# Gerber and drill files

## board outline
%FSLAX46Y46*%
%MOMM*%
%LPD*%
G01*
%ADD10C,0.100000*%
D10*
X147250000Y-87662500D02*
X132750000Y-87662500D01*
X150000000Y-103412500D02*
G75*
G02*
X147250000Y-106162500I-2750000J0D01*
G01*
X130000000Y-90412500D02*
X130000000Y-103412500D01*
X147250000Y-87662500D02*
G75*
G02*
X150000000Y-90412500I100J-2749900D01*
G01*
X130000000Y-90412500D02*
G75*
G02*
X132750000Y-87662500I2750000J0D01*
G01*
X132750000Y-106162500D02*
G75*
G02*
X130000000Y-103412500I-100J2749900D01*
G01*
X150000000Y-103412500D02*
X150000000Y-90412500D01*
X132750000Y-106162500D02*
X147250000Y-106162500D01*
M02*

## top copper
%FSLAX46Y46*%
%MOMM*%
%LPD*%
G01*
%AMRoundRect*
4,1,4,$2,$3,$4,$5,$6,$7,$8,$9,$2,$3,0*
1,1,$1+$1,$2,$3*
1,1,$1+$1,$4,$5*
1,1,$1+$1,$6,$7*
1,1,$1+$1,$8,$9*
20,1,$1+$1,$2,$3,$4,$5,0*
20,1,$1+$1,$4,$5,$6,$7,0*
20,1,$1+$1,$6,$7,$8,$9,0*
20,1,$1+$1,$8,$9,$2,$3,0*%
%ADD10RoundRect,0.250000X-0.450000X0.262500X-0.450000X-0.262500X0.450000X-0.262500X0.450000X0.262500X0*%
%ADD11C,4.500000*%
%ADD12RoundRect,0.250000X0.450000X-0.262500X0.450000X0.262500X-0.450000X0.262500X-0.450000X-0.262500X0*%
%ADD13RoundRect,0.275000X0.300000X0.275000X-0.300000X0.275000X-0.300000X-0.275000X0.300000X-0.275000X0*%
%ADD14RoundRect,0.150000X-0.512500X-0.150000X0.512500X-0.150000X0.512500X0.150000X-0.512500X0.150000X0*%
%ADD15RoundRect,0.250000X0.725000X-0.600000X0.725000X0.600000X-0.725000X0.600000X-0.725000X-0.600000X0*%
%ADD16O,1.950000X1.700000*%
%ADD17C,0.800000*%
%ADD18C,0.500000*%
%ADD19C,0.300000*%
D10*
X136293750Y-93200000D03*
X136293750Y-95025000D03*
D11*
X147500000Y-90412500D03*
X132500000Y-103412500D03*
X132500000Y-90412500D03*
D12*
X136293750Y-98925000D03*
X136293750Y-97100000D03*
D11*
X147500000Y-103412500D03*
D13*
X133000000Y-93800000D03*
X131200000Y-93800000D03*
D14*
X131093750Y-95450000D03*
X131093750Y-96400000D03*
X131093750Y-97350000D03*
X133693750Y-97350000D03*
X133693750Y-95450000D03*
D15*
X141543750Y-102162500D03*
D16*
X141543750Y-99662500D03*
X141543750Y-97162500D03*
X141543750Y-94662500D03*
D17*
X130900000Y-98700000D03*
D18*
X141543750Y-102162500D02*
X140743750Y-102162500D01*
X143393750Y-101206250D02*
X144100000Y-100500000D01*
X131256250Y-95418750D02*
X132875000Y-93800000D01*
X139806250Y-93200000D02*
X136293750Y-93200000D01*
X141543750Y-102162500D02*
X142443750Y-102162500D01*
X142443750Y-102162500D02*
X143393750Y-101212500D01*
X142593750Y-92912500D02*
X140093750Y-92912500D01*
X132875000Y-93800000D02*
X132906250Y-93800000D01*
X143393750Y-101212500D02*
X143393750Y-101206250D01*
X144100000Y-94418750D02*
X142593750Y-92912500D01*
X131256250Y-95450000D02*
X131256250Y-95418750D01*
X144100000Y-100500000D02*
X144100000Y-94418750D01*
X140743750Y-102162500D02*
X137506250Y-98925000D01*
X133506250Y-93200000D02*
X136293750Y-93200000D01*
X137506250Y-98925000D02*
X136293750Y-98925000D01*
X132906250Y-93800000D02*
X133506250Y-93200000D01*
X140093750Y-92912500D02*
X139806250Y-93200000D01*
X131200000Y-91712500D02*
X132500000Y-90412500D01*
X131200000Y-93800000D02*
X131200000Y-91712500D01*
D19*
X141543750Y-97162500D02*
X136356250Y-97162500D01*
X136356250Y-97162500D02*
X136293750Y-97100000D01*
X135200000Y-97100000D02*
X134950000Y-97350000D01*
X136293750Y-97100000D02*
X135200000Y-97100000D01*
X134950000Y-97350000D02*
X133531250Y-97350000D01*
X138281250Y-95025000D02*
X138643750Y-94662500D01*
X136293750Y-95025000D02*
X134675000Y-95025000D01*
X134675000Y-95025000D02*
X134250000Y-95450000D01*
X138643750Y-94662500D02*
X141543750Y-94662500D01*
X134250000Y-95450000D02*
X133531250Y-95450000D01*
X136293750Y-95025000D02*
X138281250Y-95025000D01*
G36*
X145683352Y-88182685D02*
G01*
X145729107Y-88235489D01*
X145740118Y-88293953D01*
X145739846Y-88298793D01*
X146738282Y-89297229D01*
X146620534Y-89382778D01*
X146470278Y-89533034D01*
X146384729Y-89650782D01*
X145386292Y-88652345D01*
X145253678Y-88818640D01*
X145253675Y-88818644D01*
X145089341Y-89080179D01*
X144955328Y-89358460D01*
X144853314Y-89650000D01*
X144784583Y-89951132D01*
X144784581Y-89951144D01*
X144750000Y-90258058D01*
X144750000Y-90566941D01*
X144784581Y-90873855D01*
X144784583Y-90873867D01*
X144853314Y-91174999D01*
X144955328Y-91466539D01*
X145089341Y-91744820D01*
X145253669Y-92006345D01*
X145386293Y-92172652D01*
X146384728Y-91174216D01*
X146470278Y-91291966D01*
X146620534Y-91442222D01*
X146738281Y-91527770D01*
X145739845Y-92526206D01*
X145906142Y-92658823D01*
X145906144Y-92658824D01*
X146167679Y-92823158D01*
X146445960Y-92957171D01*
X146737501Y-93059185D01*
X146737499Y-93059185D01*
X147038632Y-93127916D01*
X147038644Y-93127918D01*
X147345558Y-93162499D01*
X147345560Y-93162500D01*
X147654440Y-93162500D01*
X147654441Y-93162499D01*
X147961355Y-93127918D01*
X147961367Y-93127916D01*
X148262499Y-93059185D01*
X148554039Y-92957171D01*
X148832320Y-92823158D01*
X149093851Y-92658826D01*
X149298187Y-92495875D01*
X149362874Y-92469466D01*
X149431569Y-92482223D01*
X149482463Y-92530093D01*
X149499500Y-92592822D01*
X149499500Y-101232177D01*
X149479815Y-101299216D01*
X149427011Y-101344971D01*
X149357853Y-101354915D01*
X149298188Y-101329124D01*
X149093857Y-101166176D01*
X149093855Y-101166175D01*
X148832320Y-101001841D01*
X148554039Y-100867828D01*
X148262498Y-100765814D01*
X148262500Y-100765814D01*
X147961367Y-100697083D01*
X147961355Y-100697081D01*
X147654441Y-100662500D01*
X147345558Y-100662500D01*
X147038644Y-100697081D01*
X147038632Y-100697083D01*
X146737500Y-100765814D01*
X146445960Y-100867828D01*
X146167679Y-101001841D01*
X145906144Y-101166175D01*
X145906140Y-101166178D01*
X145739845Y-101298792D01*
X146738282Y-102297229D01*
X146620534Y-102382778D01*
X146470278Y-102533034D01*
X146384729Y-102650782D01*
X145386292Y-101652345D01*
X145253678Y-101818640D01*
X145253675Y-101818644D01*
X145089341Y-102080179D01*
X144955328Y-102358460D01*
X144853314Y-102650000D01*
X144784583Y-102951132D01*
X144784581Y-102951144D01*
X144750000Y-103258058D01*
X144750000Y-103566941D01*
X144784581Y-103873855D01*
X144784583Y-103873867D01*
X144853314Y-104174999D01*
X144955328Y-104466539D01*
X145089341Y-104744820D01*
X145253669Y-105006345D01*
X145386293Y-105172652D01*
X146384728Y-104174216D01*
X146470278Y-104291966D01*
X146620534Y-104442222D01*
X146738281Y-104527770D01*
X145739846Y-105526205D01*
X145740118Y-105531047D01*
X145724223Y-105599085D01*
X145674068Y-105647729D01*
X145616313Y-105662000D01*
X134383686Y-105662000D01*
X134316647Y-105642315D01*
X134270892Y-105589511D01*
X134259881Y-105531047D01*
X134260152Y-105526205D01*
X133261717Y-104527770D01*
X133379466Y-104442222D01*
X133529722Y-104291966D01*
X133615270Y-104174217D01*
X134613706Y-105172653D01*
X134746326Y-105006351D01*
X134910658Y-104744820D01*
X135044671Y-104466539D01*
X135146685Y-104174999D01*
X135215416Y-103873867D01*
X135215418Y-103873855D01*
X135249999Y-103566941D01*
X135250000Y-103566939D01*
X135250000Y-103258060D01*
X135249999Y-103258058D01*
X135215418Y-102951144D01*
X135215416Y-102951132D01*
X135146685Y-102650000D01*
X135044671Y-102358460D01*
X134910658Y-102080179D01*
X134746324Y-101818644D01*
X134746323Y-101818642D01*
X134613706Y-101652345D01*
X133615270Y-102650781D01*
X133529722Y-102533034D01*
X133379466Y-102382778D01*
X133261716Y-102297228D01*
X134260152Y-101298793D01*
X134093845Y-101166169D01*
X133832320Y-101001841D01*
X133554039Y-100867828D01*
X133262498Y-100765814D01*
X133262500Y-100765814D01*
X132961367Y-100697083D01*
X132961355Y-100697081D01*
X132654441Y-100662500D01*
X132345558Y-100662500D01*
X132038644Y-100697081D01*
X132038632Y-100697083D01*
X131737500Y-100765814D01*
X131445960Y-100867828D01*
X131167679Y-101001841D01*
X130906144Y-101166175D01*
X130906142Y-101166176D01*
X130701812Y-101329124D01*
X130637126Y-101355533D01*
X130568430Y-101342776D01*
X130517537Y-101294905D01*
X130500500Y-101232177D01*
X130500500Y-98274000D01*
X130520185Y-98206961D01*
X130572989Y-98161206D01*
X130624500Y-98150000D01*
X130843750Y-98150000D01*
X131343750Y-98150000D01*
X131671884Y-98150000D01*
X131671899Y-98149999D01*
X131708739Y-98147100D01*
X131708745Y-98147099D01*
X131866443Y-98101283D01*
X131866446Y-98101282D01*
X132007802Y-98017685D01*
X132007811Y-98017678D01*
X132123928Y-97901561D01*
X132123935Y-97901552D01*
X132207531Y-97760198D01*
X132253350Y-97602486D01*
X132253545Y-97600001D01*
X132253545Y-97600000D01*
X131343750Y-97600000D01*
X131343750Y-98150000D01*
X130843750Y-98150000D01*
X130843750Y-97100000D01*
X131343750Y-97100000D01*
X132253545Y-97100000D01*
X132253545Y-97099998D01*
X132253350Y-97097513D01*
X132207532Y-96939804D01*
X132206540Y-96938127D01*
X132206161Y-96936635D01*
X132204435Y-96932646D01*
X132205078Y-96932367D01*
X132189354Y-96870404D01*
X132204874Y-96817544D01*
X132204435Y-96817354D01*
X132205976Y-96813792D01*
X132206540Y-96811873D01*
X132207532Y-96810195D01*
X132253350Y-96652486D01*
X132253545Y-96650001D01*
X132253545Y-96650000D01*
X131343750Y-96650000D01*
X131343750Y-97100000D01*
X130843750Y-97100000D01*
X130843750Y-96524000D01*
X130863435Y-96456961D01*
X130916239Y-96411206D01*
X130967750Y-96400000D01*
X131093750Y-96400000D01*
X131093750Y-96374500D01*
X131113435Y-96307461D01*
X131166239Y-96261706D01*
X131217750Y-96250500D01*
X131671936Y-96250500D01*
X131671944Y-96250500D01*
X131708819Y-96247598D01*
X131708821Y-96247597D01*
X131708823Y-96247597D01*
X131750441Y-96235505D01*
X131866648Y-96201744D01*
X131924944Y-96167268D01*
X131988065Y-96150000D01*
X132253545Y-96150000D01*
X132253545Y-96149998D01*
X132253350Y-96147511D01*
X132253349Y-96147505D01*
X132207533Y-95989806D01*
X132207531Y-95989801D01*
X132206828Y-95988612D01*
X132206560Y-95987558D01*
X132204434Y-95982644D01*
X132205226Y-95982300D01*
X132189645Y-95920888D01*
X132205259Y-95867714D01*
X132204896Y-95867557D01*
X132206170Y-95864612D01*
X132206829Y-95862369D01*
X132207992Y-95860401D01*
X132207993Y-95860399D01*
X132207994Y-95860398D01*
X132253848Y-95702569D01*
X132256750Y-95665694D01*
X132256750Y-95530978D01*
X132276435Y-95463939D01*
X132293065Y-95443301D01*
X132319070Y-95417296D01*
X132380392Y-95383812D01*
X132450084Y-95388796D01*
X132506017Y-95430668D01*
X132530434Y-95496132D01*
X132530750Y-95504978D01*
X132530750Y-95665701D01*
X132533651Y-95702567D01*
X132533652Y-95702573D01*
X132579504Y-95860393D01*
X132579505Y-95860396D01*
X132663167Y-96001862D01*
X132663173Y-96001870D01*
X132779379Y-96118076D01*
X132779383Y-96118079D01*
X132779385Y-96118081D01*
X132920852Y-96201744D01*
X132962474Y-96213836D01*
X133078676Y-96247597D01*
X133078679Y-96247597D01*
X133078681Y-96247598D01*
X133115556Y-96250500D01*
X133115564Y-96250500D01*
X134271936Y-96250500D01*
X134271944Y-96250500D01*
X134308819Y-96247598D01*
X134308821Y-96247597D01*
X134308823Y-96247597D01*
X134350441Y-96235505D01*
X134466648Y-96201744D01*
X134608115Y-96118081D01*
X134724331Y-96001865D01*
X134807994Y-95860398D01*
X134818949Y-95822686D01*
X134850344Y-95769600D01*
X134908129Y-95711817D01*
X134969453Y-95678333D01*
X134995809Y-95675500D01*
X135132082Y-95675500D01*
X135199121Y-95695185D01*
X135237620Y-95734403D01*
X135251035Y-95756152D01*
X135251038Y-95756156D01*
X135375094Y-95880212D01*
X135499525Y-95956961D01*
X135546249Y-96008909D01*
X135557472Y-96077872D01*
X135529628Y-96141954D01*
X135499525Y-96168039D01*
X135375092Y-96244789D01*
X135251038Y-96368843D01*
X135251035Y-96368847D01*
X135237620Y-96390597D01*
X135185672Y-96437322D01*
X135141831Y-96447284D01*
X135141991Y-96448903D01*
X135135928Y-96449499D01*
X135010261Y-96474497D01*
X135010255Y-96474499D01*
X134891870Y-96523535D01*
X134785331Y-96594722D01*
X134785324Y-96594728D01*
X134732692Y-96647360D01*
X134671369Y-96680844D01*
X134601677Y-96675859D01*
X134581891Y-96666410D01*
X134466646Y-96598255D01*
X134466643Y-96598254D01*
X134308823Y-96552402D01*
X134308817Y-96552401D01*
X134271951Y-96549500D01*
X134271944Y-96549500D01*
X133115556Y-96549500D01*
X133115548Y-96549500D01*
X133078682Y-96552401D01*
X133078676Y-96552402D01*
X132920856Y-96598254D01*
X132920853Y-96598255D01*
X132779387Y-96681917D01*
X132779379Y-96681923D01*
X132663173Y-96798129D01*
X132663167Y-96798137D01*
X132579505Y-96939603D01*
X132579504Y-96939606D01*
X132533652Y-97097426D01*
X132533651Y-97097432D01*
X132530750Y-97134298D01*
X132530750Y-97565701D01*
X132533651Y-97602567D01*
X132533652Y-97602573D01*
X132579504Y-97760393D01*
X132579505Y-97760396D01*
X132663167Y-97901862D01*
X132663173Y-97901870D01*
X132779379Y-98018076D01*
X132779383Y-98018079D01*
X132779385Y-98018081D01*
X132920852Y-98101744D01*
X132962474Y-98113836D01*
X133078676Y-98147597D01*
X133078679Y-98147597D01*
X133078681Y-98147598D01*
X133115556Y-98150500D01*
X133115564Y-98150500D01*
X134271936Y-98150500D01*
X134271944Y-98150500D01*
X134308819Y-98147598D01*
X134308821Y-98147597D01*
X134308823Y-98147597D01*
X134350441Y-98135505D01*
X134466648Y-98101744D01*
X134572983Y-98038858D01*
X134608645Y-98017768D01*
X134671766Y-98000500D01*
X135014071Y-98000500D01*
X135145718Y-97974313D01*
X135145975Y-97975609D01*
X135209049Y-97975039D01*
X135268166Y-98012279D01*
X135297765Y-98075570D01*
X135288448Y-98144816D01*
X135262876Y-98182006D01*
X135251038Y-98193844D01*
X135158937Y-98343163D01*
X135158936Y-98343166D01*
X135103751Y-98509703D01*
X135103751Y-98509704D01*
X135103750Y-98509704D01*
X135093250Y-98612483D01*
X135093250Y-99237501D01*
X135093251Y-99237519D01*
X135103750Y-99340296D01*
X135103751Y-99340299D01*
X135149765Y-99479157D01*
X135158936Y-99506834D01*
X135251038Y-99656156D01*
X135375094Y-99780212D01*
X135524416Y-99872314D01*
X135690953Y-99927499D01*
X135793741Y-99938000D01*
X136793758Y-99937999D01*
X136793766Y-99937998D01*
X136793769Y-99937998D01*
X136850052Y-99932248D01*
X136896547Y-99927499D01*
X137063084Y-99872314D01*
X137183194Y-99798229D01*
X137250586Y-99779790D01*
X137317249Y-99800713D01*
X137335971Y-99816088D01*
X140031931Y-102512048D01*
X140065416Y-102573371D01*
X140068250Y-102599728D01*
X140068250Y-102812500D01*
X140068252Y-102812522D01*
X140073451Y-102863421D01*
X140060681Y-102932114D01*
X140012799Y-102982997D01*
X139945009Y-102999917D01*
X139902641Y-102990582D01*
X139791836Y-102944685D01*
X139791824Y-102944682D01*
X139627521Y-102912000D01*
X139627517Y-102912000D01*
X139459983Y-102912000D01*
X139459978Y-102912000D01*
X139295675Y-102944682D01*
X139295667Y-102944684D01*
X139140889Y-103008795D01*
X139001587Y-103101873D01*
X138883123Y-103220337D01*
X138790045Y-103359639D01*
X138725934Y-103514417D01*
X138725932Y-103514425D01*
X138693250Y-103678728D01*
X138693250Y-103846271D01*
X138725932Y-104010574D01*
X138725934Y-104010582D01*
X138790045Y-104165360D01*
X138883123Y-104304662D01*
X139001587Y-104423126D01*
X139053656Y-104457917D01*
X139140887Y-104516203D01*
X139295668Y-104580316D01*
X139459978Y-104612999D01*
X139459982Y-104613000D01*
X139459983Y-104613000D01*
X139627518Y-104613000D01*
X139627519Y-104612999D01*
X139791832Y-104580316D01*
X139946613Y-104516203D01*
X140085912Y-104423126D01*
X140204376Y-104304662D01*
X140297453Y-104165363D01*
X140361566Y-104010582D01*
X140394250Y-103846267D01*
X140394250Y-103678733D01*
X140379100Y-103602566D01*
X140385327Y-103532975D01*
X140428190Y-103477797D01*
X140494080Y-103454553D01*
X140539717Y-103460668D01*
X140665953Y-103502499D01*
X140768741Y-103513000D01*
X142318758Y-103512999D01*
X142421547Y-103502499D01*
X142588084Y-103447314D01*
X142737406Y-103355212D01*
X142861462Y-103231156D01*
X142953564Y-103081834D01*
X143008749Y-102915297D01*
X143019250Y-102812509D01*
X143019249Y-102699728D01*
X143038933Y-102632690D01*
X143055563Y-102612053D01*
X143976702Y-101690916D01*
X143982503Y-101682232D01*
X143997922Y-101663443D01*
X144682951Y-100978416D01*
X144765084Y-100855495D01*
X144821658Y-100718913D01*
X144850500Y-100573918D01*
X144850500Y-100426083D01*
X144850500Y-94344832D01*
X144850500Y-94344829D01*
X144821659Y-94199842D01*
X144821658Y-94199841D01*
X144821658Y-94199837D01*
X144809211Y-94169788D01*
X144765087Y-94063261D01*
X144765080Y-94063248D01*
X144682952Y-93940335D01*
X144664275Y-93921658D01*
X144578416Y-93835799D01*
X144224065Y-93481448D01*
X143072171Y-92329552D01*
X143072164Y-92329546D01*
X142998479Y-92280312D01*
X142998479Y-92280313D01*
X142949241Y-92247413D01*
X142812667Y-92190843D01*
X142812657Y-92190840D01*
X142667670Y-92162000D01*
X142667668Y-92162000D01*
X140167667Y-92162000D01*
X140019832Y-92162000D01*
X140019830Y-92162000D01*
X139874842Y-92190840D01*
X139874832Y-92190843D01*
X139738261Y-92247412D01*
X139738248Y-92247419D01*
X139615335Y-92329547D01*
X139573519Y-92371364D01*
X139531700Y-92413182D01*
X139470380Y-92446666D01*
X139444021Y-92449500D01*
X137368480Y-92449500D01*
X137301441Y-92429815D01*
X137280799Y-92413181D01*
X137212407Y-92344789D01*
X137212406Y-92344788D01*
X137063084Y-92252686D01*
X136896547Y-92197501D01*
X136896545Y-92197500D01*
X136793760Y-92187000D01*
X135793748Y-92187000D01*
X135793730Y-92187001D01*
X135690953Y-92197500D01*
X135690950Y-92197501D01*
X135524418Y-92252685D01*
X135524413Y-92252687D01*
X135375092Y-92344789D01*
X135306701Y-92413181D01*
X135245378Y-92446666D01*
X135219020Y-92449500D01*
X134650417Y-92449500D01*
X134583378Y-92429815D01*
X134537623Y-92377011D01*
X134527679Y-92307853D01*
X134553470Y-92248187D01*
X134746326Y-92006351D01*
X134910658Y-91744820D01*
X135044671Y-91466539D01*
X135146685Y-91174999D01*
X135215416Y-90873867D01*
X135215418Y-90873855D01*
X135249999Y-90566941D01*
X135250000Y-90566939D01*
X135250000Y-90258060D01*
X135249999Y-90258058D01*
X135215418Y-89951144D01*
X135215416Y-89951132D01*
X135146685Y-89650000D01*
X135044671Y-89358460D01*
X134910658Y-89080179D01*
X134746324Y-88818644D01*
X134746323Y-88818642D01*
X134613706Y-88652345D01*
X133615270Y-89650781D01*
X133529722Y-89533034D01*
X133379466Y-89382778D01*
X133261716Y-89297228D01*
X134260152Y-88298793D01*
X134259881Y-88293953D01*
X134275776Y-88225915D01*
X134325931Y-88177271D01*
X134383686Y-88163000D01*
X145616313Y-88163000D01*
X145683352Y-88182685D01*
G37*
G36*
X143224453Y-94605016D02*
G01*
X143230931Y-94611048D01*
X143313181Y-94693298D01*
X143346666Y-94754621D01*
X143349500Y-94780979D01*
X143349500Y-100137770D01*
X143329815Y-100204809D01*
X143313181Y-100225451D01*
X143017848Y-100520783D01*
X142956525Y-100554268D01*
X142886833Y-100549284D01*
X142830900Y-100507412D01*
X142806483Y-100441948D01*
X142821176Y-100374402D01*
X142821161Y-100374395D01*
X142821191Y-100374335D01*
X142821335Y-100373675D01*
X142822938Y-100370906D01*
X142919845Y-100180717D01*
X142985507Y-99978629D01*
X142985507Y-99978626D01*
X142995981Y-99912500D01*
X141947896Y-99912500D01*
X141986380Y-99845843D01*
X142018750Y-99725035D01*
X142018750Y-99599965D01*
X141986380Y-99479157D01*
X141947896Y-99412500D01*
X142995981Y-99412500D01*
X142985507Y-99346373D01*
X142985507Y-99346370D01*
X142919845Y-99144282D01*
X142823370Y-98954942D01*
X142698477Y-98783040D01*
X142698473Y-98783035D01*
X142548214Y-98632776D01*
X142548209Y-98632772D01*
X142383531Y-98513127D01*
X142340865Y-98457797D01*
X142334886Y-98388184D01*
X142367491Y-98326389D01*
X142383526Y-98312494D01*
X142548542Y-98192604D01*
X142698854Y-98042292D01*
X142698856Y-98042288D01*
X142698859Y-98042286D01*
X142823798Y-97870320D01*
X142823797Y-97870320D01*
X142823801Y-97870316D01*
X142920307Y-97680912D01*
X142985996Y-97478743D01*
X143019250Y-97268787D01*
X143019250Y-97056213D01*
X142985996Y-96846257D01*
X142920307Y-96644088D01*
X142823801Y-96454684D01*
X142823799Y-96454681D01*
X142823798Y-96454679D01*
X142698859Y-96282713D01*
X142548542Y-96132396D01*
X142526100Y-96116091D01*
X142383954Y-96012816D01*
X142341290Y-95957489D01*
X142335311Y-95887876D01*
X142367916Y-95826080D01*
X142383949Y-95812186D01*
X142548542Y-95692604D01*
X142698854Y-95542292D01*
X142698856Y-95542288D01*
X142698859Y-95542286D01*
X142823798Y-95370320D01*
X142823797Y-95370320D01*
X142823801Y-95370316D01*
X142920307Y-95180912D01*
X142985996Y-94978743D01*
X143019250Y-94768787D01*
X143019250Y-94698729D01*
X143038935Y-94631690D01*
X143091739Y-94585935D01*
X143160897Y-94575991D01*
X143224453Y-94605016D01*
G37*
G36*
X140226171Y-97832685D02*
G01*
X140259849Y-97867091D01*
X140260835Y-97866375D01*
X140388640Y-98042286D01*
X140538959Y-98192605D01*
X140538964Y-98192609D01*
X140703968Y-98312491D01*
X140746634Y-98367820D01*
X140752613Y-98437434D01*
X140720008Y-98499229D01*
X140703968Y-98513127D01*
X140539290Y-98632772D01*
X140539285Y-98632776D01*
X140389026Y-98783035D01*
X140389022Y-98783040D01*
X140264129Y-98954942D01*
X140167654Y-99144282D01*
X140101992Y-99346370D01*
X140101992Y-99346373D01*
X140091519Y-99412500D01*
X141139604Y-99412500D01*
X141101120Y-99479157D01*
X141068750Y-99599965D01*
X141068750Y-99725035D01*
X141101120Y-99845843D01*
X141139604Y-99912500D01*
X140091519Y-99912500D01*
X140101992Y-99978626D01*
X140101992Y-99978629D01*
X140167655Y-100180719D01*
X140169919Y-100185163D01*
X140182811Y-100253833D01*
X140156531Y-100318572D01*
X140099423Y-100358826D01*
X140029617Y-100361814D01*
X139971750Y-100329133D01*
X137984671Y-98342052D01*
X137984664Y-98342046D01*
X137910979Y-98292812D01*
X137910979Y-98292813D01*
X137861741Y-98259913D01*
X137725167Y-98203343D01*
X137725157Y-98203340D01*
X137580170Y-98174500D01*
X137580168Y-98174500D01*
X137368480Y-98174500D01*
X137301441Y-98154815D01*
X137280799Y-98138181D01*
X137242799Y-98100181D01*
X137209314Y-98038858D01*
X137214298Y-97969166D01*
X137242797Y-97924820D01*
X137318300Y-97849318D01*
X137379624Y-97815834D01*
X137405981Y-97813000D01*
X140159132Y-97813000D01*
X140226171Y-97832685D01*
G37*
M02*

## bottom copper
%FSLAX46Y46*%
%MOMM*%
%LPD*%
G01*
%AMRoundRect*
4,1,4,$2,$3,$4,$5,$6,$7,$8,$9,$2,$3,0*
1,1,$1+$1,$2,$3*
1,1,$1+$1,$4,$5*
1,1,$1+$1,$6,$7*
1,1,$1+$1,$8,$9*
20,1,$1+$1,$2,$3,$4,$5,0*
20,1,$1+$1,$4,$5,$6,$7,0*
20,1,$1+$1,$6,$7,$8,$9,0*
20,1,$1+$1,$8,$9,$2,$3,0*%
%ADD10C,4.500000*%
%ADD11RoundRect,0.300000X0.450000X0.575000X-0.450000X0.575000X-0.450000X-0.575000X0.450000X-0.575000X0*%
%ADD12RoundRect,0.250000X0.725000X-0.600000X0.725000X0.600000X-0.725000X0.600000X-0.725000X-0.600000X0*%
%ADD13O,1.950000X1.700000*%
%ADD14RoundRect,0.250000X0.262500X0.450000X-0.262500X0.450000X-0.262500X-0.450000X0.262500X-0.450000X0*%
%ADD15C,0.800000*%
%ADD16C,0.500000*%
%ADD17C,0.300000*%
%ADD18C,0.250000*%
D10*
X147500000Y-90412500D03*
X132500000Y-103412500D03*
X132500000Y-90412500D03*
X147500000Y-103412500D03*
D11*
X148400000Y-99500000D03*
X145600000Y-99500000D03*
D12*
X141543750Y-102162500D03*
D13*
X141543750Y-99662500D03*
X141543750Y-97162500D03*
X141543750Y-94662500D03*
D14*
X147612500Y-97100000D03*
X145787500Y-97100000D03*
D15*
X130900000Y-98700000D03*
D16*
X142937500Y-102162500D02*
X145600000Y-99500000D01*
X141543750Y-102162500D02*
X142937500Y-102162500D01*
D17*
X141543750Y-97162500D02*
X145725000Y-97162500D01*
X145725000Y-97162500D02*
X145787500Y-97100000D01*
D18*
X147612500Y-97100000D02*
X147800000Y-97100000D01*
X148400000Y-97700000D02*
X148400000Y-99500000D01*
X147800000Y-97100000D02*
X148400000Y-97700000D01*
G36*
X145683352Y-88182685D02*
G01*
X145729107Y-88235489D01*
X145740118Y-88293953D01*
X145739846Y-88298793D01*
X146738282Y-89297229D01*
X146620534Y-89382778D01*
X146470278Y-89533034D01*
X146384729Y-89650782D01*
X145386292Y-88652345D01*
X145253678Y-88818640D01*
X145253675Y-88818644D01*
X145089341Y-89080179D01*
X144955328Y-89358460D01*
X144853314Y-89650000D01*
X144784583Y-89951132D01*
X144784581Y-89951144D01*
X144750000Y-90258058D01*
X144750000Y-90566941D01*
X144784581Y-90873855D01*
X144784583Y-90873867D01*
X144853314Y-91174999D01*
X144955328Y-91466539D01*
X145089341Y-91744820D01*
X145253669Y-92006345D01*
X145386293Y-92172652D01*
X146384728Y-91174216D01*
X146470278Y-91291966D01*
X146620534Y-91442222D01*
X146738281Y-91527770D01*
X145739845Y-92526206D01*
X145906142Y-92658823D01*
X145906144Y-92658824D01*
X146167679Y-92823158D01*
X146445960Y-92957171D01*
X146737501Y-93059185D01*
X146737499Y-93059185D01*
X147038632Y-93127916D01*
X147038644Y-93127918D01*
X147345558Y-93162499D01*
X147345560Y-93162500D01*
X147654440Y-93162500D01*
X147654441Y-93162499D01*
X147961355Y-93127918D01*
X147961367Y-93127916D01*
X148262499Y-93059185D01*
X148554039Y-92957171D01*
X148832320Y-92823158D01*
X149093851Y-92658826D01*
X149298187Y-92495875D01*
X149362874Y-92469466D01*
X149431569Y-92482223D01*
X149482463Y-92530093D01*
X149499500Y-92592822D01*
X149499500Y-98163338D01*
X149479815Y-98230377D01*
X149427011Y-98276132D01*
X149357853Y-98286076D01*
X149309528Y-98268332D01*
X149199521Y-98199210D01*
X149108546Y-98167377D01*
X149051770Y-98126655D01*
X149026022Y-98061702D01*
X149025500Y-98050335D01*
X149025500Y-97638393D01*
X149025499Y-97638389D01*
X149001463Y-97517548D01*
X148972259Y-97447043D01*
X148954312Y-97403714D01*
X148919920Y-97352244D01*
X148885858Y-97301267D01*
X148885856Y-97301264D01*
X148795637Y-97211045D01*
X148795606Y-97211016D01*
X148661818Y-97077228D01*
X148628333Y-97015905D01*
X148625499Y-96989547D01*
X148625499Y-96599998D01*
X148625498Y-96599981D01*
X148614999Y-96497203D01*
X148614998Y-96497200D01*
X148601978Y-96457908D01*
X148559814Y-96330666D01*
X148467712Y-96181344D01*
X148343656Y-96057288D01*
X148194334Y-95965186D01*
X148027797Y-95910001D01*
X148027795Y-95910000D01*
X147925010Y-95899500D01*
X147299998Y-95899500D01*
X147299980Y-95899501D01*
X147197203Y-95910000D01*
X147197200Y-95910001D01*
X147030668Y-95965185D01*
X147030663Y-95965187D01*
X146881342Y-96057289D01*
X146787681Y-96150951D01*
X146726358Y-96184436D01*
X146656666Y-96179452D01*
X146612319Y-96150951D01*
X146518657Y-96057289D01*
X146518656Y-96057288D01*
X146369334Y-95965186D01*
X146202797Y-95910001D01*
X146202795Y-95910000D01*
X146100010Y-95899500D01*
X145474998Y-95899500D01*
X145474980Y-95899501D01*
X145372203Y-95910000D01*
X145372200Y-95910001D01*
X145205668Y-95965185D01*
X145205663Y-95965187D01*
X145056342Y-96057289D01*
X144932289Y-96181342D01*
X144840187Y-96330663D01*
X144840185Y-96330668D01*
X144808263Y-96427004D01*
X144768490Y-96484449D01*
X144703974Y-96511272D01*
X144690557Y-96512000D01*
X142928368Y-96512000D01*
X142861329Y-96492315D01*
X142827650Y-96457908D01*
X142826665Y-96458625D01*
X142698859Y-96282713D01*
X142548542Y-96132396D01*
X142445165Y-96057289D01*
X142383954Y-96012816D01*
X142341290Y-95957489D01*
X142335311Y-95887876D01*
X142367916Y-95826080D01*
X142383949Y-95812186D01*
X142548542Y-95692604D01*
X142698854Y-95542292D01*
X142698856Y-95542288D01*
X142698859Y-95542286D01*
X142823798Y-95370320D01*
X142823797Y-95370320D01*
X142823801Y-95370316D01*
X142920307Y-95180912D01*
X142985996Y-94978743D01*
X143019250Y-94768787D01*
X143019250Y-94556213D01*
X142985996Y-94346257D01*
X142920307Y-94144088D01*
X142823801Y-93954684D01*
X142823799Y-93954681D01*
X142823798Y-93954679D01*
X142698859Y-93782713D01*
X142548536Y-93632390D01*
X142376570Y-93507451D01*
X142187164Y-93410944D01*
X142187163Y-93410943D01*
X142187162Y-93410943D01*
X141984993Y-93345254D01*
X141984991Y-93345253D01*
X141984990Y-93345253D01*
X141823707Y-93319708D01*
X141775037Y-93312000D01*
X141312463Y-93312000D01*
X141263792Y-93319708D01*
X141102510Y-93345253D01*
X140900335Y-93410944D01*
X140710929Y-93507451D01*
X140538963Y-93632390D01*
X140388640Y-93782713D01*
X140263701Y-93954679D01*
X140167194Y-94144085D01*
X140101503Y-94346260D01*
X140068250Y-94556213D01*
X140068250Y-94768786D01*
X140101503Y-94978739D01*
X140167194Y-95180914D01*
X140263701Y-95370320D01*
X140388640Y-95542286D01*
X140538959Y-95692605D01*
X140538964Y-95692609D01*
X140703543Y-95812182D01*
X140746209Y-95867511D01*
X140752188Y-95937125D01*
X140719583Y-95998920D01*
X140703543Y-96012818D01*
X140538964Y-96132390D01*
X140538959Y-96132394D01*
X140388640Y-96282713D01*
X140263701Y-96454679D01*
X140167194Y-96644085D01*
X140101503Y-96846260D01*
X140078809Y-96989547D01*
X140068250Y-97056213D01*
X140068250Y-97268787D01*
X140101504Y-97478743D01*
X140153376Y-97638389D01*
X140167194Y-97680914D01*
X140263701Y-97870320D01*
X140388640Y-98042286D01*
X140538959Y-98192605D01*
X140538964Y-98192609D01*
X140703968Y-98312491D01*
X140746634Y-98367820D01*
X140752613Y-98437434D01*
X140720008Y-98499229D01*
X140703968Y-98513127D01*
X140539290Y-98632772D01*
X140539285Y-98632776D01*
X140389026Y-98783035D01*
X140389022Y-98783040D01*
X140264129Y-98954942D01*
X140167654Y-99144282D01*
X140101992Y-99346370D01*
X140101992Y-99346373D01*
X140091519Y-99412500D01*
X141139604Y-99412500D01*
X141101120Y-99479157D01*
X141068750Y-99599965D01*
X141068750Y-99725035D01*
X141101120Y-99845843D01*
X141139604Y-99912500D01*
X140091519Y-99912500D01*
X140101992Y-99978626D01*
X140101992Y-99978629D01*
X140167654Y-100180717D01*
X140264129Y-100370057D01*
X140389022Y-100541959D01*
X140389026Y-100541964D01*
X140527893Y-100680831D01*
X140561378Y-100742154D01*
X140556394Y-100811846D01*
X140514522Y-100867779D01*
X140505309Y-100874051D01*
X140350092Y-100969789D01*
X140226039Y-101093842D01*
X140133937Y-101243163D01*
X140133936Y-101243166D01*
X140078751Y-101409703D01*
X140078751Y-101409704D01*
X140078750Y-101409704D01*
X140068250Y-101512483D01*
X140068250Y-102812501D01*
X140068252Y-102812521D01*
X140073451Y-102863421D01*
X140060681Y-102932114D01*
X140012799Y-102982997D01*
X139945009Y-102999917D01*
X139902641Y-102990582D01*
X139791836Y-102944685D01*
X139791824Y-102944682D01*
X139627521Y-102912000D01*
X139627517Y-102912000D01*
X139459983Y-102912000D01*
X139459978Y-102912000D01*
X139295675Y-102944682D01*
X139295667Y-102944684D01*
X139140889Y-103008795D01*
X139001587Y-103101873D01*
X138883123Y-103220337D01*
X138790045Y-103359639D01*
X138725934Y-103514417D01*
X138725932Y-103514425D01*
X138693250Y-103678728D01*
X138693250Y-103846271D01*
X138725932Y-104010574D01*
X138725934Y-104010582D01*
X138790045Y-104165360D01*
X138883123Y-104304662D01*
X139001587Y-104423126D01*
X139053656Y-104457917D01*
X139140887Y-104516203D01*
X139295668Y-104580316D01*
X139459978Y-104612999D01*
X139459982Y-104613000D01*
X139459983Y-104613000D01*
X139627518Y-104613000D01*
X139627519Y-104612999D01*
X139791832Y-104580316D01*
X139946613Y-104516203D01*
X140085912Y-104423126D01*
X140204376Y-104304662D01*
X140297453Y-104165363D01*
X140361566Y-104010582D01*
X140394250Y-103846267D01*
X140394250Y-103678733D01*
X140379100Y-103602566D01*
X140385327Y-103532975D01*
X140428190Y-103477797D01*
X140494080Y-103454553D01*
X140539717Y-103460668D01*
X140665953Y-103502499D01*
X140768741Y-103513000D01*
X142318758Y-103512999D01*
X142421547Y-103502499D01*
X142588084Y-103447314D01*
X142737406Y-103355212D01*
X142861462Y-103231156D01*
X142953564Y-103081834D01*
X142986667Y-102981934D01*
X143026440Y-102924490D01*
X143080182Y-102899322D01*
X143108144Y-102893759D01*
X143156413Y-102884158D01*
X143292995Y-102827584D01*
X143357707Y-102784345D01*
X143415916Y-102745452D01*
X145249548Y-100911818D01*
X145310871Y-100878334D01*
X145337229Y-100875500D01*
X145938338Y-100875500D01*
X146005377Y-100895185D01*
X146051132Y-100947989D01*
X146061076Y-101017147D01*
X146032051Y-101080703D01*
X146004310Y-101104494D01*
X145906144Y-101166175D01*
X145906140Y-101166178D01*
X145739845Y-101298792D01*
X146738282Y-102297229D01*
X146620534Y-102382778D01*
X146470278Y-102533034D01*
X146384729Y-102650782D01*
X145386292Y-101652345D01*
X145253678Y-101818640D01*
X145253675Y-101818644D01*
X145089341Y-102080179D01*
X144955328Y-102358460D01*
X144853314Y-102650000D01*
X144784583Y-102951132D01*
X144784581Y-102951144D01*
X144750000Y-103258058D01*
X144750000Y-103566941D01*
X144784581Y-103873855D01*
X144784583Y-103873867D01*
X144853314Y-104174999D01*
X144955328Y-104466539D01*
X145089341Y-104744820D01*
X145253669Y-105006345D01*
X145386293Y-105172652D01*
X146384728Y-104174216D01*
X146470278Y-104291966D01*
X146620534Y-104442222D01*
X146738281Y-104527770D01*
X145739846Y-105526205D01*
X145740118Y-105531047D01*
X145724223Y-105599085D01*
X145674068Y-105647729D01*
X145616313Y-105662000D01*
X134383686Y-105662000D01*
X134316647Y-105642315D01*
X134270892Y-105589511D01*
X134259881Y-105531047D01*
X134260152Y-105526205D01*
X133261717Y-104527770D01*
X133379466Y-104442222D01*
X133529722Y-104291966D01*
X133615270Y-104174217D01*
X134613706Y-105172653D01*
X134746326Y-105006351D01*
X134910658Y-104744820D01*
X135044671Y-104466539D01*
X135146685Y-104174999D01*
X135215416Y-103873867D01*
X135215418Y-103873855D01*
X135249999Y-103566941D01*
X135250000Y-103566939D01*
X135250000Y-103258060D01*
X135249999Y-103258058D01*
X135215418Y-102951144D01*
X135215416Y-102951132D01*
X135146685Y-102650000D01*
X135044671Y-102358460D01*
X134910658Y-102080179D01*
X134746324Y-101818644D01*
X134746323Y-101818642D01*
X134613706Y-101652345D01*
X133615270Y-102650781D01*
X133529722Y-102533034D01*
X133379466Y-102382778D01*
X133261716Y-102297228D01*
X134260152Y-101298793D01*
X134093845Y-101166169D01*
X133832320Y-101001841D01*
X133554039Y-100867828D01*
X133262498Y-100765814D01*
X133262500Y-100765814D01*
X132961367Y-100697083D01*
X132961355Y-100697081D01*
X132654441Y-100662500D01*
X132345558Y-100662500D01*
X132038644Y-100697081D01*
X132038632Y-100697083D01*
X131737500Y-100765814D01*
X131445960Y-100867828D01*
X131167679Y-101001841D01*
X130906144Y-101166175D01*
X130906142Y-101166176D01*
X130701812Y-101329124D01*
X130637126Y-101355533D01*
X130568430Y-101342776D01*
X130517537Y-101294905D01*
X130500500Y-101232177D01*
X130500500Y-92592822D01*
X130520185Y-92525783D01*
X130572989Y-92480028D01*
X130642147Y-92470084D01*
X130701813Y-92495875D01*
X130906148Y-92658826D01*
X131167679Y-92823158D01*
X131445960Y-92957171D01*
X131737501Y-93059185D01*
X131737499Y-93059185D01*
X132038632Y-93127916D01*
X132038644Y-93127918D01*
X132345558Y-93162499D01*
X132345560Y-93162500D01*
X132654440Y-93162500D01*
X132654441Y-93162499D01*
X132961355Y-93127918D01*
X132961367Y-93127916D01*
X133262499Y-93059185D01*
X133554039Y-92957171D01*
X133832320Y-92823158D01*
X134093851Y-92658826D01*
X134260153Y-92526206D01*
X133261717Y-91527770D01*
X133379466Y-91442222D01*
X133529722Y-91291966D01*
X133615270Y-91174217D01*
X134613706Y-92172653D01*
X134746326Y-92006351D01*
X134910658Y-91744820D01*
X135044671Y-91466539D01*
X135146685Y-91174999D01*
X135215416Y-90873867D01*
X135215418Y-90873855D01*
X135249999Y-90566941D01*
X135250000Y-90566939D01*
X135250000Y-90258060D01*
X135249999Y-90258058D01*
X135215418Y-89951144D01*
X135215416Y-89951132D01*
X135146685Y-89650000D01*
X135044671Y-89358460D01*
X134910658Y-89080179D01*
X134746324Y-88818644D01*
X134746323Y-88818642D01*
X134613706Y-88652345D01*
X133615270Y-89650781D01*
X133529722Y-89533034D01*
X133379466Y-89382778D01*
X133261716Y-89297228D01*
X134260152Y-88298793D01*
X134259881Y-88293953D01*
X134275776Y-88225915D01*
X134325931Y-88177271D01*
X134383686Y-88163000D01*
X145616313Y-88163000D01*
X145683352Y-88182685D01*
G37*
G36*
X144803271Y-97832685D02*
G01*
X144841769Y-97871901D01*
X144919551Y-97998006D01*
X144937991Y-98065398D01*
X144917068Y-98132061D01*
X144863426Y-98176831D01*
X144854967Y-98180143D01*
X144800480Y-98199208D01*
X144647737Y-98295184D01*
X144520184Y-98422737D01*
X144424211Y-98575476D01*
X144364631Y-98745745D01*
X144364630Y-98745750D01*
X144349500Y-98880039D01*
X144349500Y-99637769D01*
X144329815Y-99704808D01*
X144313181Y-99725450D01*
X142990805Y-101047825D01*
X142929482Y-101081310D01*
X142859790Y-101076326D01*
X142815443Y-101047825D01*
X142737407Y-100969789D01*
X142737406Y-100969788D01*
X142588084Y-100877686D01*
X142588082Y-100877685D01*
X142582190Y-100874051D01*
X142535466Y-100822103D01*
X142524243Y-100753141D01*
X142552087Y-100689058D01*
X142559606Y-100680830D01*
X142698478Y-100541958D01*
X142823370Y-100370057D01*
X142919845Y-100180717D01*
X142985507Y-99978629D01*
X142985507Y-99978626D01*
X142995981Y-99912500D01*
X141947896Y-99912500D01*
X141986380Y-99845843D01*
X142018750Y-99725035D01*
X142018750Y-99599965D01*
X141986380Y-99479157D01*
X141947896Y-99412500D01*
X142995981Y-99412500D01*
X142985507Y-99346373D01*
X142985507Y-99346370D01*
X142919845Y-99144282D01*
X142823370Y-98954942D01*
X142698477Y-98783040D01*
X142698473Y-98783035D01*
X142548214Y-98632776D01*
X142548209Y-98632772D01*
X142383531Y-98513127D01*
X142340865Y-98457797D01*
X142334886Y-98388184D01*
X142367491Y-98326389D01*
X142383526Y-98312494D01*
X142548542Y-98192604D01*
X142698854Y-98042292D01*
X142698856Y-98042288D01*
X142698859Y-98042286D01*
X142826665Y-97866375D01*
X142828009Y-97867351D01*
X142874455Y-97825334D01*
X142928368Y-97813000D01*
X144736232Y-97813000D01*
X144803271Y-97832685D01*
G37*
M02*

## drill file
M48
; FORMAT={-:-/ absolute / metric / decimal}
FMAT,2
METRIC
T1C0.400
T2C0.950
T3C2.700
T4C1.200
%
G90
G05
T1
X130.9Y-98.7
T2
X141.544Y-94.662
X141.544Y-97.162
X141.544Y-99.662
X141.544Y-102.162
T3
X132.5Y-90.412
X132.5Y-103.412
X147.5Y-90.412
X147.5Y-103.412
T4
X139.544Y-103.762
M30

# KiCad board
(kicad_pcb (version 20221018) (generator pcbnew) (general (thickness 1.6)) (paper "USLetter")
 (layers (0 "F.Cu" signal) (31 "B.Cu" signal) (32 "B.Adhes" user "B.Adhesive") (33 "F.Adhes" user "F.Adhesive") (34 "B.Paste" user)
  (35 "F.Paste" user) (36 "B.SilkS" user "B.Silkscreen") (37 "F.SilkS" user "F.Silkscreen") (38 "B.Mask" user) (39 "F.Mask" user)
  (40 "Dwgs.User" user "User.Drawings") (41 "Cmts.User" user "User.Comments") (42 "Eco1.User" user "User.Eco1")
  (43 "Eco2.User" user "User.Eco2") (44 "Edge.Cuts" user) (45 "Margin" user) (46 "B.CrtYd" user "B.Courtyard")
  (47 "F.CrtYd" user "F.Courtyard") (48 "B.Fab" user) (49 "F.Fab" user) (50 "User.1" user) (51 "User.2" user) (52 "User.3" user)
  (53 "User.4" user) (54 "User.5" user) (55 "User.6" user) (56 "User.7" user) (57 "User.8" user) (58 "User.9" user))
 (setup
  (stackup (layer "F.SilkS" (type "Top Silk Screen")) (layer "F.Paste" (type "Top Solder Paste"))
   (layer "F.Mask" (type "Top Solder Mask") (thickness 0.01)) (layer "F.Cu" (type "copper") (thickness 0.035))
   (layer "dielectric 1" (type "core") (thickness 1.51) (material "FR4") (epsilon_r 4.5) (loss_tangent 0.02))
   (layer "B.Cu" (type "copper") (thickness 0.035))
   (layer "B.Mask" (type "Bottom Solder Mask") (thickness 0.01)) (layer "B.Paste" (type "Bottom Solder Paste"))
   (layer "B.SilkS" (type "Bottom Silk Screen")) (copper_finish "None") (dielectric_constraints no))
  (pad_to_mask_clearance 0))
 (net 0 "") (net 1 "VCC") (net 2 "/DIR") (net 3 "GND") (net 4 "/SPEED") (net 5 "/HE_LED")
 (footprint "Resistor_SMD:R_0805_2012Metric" (layer "F.Cu") (at 136.29375 94.1125 -90)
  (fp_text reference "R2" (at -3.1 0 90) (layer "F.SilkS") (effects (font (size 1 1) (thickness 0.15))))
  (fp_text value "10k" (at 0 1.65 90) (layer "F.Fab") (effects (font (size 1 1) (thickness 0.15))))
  (pad "1" smd roundrect (at -0.9125 0 270) (size 1.025 1.4) (layers "F.Cu" "F.Paste" "F.Mask") (roundrect_rratio 0.243902439) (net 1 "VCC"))
  (pad "2" smd roundrect (at 0.9125 0 270) (size 1.025 1.4) (layers "F.Cu" "F.Paste" "F.Mask") (roundrect_rratio 0.243902439) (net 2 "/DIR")))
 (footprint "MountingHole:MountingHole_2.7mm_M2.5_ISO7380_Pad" (layer "F.Cu") (at 147.5 90.4125)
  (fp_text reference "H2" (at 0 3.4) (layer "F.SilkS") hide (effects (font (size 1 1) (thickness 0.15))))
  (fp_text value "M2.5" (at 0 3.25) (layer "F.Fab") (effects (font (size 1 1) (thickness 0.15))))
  (pad "1" thru_hole circle (at 0 0) (size 4.5 4.5) (drill 2.7) (layers "*.Cu" "*.Mask") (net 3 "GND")))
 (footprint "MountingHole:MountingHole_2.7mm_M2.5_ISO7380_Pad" (layer "F.Cu") (at 132.5 103.4125)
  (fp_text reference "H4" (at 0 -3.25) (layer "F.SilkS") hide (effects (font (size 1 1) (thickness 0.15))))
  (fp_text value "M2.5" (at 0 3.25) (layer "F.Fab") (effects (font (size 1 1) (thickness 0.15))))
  (pad "1" thru_hole circle (at 0 0) (size 4.5 4.5) (drill 2.7) (layers "*.Cu" "*.Mask") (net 3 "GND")))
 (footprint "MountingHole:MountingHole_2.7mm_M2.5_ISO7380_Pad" (layer "F.Cu") (at 132.5 90.4125)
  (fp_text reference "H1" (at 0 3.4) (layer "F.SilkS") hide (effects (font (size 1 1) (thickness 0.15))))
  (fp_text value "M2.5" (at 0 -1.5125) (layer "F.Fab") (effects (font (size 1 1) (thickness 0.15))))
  (pad "1" thru_hole circle (at 0 0) (size 4.5 4.5) (drill 2.7) (layers "*.Cu" "*.Mask") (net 3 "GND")))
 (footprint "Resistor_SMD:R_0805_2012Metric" (layer "F.Cu") (at 136.29375 98.0125 90)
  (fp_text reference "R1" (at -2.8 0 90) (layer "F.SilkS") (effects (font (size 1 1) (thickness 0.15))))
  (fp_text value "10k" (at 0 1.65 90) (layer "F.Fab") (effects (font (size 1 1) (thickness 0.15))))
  (pad "1" smd roundrect (at -0.9125 0 90) (size 1.025 1.4) (layers "F.Cu" "F.Paste" "F.Mask") (roundrect_rratio 0.243902439) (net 1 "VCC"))
  (pad "2" smd roundrect (at 0.9125 0 90) (size 1.025 1.4) (layers "F.Cu" "F.Paste" "F.Mask") (roundrect_rratio 0.243902439)
   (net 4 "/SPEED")))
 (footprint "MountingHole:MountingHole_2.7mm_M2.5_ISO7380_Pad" (layer "F.Cu") (at 147.5 103.4125)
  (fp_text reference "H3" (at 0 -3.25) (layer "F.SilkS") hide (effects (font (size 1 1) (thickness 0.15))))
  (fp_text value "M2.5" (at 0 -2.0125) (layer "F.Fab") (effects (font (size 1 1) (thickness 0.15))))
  (pad "1" thru_hole circle (at 0 0) (size 4.5 4.5) (drill 2.7) (layers "*.Cu" "*.Mask") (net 3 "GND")))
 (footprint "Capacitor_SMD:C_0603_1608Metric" (layer "F.Cu") (at 132.1 93.8 180)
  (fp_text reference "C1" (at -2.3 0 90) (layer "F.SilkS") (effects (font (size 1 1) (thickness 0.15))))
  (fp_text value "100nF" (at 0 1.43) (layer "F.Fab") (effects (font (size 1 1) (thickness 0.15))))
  (pad "1" smd roundrect (at -0.9 0 180) (size 1.15 1.1) (layers "F.Cu" "F.Paste" "F.Mask") (roundrect_rratio 0.25) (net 1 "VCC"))
  (pad "2" smd roundrect (at 0.9 0 180) (size 1.15 1.1) (layers "F.Cu" "F.Paste" "F.Mask") (roundrect_rratio 0.25) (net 3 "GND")))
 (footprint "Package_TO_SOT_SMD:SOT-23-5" (layer "F.Cu") (at 132.39375 96.4)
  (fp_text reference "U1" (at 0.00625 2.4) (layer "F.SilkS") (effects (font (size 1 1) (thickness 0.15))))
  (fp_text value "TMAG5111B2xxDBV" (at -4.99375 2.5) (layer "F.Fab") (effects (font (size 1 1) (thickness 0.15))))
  (pad "1" smd roundrect (at -1.3 -0.95) (size 1.325 0.6) (layers "F.Cu" "F.Paste" "F.Mask") (roundrect_rratio 0.25) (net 1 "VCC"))
  (pad "2" smd roundrect (at -1.3 0) (size 1.325 0.6) (layers "F.Cu" "F.Paste" "F.Mask") (roundrect_rratio 0.25) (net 3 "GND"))
  (pad "3" smd roundrect (at -1.3 0.95) (size 1.325 0.6) (layers "F.Cu" "F.Paste" "F.Mask") (roundrect_rratio 0.25) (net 3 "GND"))
  (pad "4" smd roundrect (at 1.3 0.95) (size 1.325 0.6) (layers "F.Cu" "F.Paste" "F.Mask") (roundrect_rratio 0.25) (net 4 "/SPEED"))
  (pad "5" smd roundrect (at 1.3 -0.95) (size 1.325 0.6) (layers "F.Cu" "F.Paste" "F.Mask") (roundrect_rratio 0.25) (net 2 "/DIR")))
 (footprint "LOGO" (layer "F.Cu") (at 147.5 98 90)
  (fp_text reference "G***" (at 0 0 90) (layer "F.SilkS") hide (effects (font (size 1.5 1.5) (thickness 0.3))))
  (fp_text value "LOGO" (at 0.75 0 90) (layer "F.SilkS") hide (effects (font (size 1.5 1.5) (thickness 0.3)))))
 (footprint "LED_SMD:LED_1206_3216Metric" (layer "B.Cu") (at 147 99.5 180)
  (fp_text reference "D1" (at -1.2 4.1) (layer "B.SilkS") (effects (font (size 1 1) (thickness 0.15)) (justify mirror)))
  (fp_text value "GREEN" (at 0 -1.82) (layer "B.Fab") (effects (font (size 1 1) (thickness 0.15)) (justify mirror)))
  (pad "1" smd roundrect (at -1.4 0 180) (size 1.5 1.75) (layers "B.Cu" "B.Paste" "B.Mask") (roundrect_rratio 0.2) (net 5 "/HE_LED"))
  (pad "2" smd roundrect (at 1.4 0 180) (size 1.5 1.75) (layers "B.Cu" "B.Paste" "B.Mask") (roundrect_rratio 0.2) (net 1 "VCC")))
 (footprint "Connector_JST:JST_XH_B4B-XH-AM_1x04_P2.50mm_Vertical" (layer "B.Cu") (at 141.54375 102.1625 90)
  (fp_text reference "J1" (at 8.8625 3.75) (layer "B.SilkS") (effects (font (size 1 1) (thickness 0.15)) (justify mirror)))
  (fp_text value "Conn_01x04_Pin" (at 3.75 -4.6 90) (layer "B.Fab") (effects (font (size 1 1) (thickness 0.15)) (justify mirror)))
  (pad "" np_thru_hole circle (at -1.6 -2 90) (size 1.2 1.2) (drill 1.2) (layers "*.Cu" "*.Mask"))
  (pad "1" thru_hole roundrect (at 0 0 90) (size 1.7 1.95) (drill 0.95) (layers "*.Cu" "*.Mask") (roundrect_rratio 0.1470588235)
   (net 1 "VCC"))
  (pad "2" thru_hole oval (at 2.5 0 90) (size 1.7 1.95) (drill 0.95) (layers "*.Cu" "*.Mask") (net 3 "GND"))
  (pad "3" thru_hole oval (at 5 0 90) (size 1.7 1.95) (drill 0.95) (layers "*.Cu" "*.Mask") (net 4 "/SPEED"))
  (pad "4" thru_hole oval (at 7.5 0 90) (size 1.7 1.95) (drill 0.95) (layers "*.Cu" "*.Mask") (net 2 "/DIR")))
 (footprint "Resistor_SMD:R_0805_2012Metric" (layer "B.Cu") (at 146.7 97.1 180)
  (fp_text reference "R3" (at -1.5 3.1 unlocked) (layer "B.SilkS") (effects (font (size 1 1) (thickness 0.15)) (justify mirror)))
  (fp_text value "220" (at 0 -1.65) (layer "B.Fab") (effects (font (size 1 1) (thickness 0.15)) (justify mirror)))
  (pad "1" smd roundrect (at -0.9125 0 180) (size 1.025 1.4) (layers "B.Cu" "B.Paste" "B.Mask") (roundrect_rratio 0.243902439)
   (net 5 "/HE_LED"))
  (pad "2" smd roundrect (at 0.9125 0 180) (size 1.025 1.4) (layers "B.Cu" "B.Paste" "B.Mask") (roundrect_rratio 0.243902439)
   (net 4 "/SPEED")))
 (gr_line (start 147.25 87.6625) (end 132.75 87.6625) (stroke (width 0.1) (type default)) (layer "Edge.Cuts"))
 (gr_arc (start 150 103.4125) (mid 149.194541 105.357026) (end 147.25 106.1625) (stroke (width 0.1) (type default)) (layer "Edge.Cuts"))
 (gr_line (start 130 90.4125) (end 130 103.4125) (stroke (width 0.1) (type default)) (layer "Edge.Cuts"))
 (gr_arc (start 147.25 87.6625) (mid 149.194576 88.467939) (end 150 90.4125) (stroke (width 0.1) (type default)) (layer "Edge.Cuts"))
 (gr_arc (start 130 90.4125) (mid 130.805459 88.467974) (end 132.75 87.6625) (stroke (width 0.1) (type default)) (layer "Edge.Cuts"))
 (gr_arc (start 132.75 106.1625) (mid 130.805424 105.357061) (end 130 103.4125) (stroke (width 0.1) (type default)) (layer "Edge.Cuts"))
 (gr_line (start 150 103.4125) (end 150 90.4125) (stroke (width 0.1) (type default)) (layer "Edge.Cuts"))
 (gr_line (start 132.75 106.1625) (end 147.25 106.1625) (stroke (width 0.1) (type default)) (layer "Edge.Cuts"))
 (segment (start 141.54375 102.1625) (end 140.74375 102.1625) (width 0.5) (layer "F.Cu") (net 1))
 (segment (start 143.39375 101.20625) (end 144.1 100.5) (width 0.5) (layer "F.Cu") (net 1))
 (segment (start 131.25625 95.41875) (end 132.875 93.8) (width 0.5) (layer "F.Cu") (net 1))
 (segment (start 139.80625 93.2) (end 136.29375 93.2) (width 0.5) (layer "F.Cu") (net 1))
 (segment (start 141.54375 102.1625) (end 142.44375 102.1625) (width 0.5) (layer "F.Cu") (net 1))
 (segment (start 142.44375 102.1625) (end 143.39375 101.2125) (width 0.5) (layer "F.Cu") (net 1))
 (segment (start 142.59375 92.9125) (end 140.09375 92.9125) (width 0.5) (layer "F.Cu") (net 1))
 (segment (start 132.875 93.8) (end 132.90625 93.8) (width 0.5) (layer "F.Cu") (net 1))
 (segment (start 143.39375 101.2125) (end 143.39375 101.20625) (width 0.5) (layer "F.Cu") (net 1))
 (segment (start 144.1 94.41875) (end 142.59375 92.9125) (width 0.5) (layer "F.Cu") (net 1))
 (segment (start 131.25625 95.45) (end 131.25625 95.41875) (width 0.5) (layer "F.Cu") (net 1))
 (segment (start 144.1 100.5) (end 144.1 94.41875) (width 0.5) (layer "F.Cu") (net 1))
 (segment (start 140.74375 102.1625) (end 137.50625 98.925) (width 0.5) (layer "F.Cu") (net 1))
 (segment (start 133.50625 93.2) (end 136.29375 93.2) (width 0.5) (layer "F.Cu") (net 1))
 (segment (start 137.50625 98.925) (end 136.29375 98.925) (width 0.5) (layer "F.Cu") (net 1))
 (segment (start 132.90625 93.8) (end 133.50625 93.2) (width 0.5) (layer "F.Cu") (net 1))
 (segment (start 140.09375 92.9125) (end 139.80625 93.2) (width 0.5) (layer "F.Cu") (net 1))
 (segment (start 142.9375 102.1625) (end 145.6 99.5) (width 0.5) (layer "B.Cu") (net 1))
 (segment (start 141.54375 102.1625) (end 142.9375 102.1625) (width 0.5) (layer "B.Cu") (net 1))
 (segment (start 131.2 91.7125) (end 132.5 90.4125) (width 0.5) (layer "F.Cu") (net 3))
 (segment (start 131.2 93.8) (end 131.2 91.7125) (width 0.5) (layer "F.Cu") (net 3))
 (via (at 130.9 98.7) (size 0.8) (drill 0.4) (layers "F.Cu" "B.Cu") (free) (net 3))
 (segment (start 141.54375 97.1625) (end 136.35625 97.1625) (width 0.3) (layer "F.Cu") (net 4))
 (segment (start 136.35625 97.1625) (end 136.29375 97.1) (width 0.3) (layer "F.Cu") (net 4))
 (segment (start 135.2 97.1) (end 134.95 97.35) (width 0.3) (layer "F.Cu") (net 4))
 (segment (start 136.29375 97.1) (end 135.2 97.1) (width 0.3) (layer "F.Cu") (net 4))
 (segment (start 134.95 97.35) (end 133.53125 97.35) (width 0.3) (layer "F.Cu") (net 4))
 (segment (start 141.54375 97.1625) (end 145.725 97.1625) (width 0.3) (layer "B.Cu") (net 4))
 (segment (start 145.725 97.1625) (end 145.7875 97.1) (width 0.3) (layer "B.Cu") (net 4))
 (segment (start 138.28125 95.025) (end 138.64375 94.6625) (width 0.3) (layer "F.Cu") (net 2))
 (segment (start 136.29375 95.025) (end 134.675 95.025) (width 0.3) (layer "F.Cu") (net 2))
 (segment (start 134.675 95.025) (end 134.25 95.45) (width 0.3) (layer "F.Cu") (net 2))
 (segment (start 138.64375 94.6625) (end 141.54375 94.6625) (width 0.3) (layer "F.Cu") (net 2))
 (segment (start 134.25 95.45) (end 133.53125 95.45) (width 0.3) (layer "F.Cu") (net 2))
 (segment (start 136.29375 95.025) (end 138.28125 95.025) (width 0.3) (layer "F.Cu") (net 2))
 (segment (start 147.6125 97.1) (end 147.8 97.1) (width 0.25) (layer "B.Cu") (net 5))
 (segment (start 148.4 97.7) (end 148.4 99.5) (width 0.25) (layer "B.Cu") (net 5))
 (segment (start 147.8 97.1) (end 148.4 97.7) (width 0.25) (layer "B.Cu") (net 5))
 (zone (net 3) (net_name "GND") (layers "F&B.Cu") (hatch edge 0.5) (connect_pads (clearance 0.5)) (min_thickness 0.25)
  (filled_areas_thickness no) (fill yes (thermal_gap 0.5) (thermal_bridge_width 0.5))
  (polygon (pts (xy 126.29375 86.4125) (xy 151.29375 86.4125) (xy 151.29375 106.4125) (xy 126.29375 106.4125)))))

